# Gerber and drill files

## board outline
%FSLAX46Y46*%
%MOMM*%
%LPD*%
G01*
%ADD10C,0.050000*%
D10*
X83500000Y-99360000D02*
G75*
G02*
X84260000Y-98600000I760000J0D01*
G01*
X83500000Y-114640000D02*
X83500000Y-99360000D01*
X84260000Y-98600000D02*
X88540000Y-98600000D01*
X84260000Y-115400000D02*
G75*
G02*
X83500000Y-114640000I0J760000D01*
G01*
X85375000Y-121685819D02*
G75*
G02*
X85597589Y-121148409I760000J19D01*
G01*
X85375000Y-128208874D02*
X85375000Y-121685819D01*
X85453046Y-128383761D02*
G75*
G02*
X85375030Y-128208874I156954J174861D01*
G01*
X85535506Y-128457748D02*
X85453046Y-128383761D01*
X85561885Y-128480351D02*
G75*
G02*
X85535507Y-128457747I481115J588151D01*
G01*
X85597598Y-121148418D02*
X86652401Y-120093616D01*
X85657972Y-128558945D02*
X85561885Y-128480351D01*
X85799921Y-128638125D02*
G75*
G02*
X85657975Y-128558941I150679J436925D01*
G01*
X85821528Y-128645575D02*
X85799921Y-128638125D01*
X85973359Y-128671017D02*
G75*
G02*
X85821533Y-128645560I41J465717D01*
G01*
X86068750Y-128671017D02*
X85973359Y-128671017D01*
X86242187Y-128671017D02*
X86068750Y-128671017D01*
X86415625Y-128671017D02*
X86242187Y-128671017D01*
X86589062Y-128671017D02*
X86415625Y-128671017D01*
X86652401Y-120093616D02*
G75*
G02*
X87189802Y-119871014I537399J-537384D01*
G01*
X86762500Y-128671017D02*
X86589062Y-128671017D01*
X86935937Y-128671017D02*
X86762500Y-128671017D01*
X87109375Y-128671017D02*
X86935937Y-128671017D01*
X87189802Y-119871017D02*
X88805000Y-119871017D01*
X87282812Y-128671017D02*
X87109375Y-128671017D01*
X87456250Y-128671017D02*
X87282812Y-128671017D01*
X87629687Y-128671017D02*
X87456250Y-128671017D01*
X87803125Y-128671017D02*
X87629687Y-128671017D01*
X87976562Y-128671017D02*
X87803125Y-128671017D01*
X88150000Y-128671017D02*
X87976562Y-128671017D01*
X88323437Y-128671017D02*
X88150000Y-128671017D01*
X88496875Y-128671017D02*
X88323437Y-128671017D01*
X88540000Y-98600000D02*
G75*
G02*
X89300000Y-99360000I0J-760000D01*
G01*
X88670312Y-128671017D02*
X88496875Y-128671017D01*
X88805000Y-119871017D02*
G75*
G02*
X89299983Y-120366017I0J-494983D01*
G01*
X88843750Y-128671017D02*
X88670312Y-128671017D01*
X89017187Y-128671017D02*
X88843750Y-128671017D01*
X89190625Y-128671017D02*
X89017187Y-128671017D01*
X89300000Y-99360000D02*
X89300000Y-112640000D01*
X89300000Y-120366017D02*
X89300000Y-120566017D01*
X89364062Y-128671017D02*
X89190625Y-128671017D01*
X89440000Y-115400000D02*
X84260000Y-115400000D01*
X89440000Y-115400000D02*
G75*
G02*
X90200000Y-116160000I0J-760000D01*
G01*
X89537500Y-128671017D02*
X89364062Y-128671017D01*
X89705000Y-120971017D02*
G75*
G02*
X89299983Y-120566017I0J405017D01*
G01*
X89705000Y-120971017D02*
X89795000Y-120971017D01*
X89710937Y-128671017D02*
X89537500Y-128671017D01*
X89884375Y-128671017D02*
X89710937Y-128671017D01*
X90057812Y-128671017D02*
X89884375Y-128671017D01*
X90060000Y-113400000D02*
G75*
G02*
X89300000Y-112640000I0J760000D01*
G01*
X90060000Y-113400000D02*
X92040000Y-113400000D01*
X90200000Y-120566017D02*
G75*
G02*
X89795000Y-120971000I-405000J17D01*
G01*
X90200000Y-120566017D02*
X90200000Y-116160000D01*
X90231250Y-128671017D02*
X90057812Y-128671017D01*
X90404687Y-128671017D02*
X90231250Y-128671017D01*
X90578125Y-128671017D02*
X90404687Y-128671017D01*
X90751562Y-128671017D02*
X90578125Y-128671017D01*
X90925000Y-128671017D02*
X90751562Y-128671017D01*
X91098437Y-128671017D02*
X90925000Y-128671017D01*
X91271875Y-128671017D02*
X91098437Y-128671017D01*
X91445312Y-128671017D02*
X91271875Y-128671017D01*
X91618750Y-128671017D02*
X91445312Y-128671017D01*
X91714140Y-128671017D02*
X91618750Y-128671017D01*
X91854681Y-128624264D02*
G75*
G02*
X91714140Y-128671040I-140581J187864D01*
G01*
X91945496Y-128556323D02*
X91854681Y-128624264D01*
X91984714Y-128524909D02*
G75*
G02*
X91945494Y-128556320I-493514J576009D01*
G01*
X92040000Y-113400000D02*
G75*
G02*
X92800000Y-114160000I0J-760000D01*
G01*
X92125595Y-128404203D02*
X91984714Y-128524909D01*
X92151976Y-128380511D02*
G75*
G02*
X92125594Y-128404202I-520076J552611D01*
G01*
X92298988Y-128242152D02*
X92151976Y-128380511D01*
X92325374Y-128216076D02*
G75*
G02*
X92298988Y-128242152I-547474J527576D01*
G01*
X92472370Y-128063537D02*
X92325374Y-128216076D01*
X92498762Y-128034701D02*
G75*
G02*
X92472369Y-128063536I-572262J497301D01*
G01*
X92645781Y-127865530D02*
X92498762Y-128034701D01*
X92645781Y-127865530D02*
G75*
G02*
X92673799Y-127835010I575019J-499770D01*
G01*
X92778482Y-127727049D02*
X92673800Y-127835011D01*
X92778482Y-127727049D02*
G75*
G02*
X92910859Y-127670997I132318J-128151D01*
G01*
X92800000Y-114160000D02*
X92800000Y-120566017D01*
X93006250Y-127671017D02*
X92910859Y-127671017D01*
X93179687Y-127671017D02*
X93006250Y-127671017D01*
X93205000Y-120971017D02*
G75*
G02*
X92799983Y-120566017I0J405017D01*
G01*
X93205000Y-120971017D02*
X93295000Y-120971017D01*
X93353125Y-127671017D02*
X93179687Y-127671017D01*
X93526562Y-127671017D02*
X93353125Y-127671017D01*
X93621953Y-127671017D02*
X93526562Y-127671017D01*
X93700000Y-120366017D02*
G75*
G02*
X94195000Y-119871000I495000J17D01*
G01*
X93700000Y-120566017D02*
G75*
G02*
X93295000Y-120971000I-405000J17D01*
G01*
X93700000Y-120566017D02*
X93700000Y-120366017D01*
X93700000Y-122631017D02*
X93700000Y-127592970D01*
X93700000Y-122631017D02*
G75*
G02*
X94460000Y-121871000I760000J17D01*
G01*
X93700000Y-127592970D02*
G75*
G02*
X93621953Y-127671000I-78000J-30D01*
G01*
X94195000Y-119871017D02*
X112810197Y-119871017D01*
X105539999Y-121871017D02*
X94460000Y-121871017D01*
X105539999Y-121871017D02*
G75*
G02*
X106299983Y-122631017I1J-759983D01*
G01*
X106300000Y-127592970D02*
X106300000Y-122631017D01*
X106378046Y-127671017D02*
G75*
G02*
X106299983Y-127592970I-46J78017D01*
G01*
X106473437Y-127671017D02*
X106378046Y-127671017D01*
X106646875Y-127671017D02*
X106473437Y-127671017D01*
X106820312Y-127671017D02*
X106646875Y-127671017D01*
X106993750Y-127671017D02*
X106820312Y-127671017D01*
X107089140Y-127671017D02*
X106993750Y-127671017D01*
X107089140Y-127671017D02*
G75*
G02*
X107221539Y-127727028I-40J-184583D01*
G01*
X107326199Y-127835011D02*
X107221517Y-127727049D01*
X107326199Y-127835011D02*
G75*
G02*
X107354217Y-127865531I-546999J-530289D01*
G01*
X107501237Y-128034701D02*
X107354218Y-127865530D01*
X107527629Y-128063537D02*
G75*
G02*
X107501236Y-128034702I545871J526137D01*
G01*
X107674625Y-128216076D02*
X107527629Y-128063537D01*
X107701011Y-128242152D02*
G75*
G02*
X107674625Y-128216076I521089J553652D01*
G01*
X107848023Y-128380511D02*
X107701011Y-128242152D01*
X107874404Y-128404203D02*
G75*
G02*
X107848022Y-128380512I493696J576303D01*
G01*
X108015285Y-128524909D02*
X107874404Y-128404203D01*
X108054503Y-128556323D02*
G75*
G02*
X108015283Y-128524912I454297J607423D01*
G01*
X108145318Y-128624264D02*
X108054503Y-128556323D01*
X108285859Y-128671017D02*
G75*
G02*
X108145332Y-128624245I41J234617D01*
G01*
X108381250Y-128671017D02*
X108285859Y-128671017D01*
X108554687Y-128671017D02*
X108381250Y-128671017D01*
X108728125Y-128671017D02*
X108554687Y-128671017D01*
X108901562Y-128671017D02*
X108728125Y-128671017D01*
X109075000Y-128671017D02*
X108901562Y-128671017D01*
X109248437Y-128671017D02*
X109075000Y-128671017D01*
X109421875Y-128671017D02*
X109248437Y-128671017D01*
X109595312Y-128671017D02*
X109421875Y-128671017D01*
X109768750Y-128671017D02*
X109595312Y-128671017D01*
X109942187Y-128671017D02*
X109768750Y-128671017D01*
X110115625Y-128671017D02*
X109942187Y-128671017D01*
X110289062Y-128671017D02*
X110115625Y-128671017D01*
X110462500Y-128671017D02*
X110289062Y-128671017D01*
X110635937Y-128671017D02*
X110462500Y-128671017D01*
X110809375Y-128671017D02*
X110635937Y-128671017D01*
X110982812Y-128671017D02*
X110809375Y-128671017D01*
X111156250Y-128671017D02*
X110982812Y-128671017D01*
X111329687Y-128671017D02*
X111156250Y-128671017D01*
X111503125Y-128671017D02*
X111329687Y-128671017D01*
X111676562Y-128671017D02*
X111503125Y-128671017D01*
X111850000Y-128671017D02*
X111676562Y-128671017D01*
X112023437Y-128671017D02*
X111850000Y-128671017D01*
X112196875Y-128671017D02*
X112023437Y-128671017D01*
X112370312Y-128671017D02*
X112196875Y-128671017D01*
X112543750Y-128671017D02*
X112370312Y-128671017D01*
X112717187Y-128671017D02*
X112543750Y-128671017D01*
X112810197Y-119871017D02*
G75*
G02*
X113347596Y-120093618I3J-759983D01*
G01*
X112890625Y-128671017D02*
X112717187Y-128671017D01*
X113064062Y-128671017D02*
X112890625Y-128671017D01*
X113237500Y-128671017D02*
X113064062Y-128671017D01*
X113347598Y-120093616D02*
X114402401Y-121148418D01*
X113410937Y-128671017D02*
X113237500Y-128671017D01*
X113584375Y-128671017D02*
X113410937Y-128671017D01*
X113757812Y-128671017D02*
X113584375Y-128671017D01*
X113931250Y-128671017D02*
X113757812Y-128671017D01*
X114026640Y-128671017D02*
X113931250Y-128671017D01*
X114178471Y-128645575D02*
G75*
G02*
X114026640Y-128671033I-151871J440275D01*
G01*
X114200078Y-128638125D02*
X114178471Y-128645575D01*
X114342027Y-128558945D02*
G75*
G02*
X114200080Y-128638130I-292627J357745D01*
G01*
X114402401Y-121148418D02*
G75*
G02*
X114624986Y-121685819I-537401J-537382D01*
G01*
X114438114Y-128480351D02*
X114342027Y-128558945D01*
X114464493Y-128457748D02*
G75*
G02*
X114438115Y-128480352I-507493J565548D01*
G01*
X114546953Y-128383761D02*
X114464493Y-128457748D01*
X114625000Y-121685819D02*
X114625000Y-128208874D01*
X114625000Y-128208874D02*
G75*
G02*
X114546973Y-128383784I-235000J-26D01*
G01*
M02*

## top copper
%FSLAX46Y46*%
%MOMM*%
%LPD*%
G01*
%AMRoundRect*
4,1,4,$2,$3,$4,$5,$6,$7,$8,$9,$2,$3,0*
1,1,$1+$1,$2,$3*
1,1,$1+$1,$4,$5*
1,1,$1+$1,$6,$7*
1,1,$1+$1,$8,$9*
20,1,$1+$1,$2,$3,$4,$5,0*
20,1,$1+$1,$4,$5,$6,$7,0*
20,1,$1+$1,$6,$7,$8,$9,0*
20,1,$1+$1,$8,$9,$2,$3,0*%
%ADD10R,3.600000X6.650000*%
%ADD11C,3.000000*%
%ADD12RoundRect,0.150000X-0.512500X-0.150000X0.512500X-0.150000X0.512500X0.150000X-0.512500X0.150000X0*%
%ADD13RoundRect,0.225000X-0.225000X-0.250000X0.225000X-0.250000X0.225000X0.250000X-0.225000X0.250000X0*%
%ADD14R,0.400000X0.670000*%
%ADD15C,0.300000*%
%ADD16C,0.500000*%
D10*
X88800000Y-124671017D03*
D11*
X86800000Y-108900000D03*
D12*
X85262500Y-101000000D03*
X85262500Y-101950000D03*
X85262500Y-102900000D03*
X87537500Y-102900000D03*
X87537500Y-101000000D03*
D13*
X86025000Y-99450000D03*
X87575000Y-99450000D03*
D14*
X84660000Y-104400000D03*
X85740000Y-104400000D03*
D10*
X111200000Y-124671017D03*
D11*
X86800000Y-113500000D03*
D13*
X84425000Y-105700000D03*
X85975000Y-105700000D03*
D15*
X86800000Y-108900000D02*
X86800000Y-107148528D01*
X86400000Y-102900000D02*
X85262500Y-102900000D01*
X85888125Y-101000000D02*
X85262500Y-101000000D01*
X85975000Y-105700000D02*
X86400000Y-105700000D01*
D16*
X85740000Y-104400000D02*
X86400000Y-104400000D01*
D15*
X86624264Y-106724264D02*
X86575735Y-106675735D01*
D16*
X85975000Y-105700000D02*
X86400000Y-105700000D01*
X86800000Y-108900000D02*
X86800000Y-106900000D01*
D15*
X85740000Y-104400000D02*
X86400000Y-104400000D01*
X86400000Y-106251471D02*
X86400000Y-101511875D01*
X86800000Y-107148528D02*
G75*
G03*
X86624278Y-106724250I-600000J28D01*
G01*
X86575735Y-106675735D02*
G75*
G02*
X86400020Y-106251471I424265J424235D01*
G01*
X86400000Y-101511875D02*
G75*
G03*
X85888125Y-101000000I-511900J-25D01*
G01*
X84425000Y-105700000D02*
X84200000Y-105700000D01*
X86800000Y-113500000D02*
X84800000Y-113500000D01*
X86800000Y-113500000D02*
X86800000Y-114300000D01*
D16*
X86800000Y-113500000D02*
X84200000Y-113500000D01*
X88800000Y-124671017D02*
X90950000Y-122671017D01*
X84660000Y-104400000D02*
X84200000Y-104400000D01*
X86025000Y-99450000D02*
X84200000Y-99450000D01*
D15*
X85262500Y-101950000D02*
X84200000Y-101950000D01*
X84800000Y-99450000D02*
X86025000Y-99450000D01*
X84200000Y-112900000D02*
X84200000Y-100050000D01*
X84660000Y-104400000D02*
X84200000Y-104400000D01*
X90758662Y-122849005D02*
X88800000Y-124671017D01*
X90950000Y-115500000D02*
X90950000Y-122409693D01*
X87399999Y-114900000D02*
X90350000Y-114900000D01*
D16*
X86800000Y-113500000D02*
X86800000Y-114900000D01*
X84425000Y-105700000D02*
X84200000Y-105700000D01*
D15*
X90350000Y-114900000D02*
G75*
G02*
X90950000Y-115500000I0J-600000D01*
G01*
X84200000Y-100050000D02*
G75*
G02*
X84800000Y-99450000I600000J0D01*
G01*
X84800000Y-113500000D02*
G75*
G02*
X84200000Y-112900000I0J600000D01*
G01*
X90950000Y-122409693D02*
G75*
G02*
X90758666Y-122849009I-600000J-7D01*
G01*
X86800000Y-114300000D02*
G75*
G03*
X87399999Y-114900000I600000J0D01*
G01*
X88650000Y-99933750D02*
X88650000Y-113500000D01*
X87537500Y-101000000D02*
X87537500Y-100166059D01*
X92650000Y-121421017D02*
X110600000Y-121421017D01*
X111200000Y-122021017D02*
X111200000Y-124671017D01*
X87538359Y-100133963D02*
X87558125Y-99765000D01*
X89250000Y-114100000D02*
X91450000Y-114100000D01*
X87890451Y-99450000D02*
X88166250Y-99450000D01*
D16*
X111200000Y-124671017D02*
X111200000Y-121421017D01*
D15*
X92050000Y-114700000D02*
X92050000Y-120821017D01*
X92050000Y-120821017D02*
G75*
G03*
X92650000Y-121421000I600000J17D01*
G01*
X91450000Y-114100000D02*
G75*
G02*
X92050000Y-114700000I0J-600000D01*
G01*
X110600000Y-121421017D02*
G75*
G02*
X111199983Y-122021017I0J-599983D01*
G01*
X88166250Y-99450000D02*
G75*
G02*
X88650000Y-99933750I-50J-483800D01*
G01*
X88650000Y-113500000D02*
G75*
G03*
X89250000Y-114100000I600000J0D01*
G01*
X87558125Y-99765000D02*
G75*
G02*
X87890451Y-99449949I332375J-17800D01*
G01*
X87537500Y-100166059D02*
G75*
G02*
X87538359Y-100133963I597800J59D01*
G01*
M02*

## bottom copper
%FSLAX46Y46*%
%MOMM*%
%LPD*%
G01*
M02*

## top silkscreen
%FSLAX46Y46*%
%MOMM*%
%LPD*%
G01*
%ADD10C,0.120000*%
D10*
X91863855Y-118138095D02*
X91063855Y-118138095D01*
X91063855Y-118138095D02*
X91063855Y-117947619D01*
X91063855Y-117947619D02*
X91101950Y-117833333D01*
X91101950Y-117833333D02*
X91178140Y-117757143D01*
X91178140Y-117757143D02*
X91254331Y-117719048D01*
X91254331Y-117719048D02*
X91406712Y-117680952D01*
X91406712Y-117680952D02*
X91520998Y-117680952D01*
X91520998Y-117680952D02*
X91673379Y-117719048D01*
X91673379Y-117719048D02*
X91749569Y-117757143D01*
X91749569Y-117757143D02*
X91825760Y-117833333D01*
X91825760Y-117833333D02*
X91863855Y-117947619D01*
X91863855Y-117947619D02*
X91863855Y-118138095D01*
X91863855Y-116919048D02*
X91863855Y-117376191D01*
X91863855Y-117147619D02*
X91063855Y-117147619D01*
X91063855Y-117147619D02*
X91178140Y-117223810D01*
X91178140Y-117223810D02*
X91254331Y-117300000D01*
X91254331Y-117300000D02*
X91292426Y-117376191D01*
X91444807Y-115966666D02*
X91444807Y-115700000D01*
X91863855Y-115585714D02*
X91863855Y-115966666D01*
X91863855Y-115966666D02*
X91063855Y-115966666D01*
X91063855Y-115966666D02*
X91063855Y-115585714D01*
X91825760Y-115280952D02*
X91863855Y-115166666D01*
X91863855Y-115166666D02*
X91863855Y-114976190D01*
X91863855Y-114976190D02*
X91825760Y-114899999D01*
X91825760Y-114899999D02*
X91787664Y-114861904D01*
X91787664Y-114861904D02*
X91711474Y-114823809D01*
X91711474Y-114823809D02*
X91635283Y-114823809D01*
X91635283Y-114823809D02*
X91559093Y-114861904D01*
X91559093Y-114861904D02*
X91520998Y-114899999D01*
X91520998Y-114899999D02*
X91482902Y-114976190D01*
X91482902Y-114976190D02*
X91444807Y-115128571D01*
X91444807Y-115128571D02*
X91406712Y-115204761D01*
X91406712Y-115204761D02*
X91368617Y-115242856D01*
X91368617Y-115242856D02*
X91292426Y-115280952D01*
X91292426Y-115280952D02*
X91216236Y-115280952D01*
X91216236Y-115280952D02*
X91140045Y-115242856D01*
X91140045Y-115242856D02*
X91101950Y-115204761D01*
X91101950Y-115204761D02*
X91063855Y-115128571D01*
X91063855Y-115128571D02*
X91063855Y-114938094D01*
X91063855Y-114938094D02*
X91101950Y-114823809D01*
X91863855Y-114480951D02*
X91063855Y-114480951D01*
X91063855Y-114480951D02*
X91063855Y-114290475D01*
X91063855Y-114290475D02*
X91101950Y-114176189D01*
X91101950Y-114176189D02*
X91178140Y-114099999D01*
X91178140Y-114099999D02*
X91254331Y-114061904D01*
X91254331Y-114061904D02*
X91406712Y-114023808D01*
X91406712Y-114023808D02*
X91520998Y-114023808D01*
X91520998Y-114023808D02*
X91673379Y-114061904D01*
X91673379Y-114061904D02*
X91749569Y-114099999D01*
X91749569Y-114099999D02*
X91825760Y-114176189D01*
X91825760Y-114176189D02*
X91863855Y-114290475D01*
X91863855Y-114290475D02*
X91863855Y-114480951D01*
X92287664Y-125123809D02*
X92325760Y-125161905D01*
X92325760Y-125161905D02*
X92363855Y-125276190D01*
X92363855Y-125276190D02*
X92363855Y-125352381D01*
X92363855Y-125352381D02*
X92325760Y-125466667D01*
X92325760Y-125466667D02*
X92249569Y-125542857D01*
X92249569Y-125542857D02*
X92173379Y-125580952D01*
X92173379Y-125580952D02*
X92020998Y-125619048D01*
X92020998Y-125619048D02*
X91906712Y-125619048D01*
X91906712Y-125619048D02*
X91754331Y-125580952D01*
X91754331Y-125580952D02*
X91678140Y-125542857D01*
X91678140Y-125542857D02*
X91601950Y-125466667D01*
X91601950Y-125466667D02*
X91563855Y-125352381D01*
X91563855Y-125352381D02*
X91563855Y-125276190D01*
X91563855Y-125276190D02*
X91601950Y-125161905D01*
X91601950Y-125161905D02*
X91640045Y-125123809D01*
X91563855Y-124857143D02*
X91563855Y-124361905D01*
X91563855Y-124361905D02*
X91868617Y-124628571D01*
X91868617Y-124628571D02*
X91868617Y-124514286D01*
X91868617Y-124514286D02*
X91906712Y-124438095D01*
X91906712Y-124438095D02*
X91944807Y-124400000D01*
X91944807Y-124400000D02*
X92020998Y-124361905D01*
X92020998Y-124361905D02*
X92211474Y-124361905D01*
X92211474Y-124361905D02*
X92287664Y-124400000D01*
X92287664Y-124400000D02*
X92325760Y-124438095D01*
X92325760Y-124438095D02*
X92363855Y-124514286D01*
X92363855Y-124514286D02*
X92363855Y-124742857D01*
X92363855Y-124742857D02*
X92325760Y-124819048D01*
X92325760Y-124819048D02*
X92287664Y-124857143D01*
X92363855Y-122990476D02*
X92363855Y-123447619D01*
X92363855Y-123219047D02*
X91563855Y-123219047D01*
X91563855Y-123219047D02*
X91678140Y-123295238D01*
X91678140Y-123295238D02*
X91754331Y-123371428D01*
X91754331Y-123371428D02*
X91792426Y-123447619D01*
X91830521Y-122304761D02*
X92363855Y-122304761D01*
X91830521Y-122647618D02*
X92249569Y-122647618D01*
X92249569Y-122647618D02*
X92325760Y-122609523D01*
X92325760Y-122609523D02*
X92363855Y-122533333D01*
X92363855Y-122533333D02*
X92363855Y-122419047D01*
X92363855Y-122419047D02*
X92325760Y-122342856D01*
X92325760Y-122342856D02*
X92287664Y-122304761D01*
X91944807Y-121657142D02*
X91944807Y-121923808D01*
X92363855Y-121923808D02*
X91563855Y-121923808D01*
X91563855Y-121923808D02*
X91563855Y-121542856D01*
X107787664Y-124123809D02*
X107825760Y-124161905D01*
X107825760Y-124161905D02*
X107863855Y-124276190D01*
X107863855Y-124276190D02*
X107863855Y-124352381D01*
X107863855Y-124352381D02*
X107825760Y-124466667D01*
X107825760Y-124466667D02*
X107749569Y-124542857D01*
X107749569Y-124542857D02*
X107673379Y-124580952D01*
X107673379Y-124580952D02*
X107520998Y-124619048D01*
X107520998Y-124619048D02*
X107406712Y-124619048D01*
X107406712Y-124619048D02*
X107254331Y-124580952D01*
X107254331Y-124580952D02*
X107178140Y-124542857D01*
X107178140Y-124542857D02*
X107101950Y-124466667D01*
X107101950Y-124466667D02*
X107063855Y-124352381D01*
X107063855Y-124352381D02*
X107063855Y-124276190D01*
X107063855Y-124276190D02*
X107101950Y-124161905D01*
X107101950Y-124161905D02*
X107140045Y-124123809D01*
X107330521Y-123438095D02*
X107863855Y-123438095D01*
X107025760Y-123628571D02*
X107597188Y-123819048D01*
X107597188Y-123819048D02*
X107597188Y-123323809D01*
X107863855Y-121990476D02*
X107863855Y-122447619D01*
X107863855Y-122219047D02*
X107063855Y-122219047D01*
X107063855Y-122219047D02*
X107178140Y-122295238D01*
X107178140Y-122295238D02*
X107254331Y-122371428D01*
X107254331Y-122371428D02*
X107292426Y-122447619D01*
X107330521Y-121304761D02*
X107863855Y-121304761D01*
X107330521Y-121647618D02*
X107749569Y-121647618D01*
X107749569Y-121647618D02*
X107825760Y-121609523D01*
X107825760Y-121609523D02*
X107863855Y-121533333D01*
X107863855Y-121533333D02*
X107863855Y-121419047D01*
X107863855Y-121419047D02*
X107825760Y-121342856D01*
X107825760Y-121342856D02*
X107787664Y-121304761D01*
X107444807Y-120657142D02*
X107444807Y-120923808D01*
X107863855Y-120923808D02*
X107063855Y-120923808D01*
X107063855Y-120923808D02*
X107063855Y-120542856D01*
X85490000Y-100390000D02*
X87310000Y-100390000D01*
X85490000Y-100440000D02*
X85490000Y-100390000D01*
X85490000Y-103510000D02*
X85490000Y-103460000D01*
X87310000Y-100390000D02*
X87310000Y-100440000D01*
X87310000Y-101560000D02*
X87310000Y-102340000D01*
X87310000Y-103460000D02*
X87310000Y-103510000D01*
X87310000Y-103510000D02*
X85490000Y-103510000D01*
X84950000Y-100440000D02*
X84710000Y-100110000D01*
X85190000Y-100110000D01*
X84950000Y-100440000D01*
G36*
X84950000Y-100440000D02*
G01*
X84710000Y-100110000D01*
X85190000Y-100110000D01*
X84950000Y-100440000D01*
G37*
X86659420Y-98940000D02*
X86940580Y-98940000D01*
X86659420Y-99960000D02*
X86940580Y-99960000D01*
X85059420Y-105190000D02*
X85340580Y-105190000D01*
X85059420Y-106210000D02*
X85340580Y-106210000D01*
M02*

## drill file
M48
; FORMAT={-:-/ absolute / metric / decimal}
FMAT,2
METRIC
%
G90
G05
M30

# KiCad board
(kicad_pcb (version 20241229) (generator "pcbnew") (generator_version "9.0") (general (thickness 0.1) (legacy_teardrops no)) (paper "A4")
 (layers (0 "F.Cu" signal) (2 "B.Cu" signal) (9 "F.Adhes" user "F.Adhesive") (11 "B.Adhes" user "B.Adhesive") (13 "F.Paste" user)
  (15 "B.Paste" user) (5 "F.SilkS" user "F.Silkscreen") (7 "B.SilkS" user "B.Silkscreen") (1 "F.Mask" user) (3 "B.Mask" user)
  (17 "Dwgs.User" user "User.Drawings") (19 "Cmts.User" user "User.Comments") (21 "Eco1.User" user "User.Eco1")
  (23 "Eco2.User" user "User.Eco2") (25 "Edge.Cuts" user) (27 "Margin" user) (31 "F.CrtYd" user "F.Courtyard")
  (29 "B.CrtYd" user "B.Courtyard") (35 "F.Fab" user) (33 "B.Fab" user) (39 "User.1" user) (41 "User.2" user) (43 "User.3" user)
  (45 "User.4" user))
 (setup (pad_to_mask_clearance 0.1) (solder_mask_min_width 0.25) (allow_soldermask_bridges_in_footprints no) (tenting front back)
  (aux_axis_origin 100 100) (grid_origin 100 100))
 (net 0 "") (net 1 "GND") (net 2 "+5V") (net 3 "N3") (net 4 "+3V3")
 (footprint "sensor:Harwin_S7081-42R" (layer "F.Cu") (at 88.8 124.671017 90)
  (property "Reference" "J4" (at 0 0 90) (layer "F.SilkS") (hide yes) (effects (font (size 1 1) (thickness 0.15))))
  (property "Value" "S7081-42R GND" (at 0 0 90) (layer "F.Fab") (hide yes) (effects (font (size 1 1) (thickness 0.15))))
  (pad "1" smd rect (at 0 0 90) (size 6.65 3.6) (layers "F.Cu" "F.Mask" "F.Paste") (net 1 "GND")))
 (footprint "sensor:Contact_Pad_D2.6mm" (layer "F.Cu") (at 86.8 108.9)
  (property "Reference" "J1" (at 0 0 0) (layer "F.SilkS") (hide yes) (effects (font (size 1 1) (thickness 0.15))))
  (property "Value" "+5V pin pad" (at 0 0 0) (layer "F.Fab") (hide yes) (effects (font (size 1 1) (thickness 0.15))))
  (pad "1" smd circle (at 0 0) (size 3 3) (layers "F.Cu" "F.Mask") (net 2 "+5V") (solder_mask_margin -0.2)))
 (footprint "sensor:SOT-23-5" (layer "F.Cu") (at 86.4 101.95)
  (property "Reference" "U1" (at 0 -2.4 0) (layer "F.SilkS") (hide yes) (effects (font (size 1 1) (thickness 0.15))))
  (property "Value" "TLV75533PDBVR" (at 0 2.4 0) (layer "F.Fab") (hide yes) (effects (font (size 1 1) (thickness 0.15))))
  (fp_line (start -0.91 -1.56) (end 0.91 -1.56) (stroke (width 0.12) (type solid)) (layer "F.SilkS"))
  (fp_line (start -0.91 -1.51) (end -0.91 -1.56) (stroke (width 0.12) (type solid)) (layer "F.SilkS"))
  (fp_line (start -0.91 1.56) (end -0.91 1.51) (stroke (width 0.12) (type solid)) (layer "F.SilkS"))
  (fp_line (start 0.91 -1.56) (end 0.91 -1.51) (stroke (width 0.12) (type solid)) (layer "F.SilkS"))
  (fp_line (start 0.91 -0.39) (end 0.91 0.39) (stroke (width 0.12) (type solid)) (layer "F.SilkS"))
  (fp_line (start 0.91 1.51) (end 0.91 1.56) (stroke (width 0.12) (type solid)) (layer "F.SilkS"))
  (fp_line (start 0.91 1.56) (end -0.91 1.56) (stroke (width 0.12) (type solid)) (layer "F.SilkS"))
  (fp_poly (pts (xy -1.45 -1.51) (xy -1.69 -1.84) (xy -1.21 -1.84)) (stroke (width 0.12) (type solid)) (fill yes) (layer "F.SilkS"))
  (pad "1" smd roundrect (at -1.1375 -0.95) (size 1.325 0.6) (layers "F.Cu" "F.Mask" "F.Paste") (roundrect_rratio 0.25) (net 2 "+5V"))
  (pad "2" smd roundrect (at -1.1375 0) (size 1.325 0.6) (layers "F.Cu" "F.Mask" "F.Paste") (roundrect_rratio 0.25) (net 1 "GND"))
  (pad "3" smd roundrect (at -1.1375 0.95) (size 1.325 0.6) (layers "F.Cu" "F.Mask" "F.Paste") (roundrect_rratio 0.25) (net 2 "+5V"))
  (pad "4" smd roundrect (at 1.1375 0.95) (size 1.325 0.6) (layers "F.Cu" "F.Mask" "F.Paste") (roundrect_rratio 0.25) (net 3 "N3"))
  (pad "5" smd roundrect (at 1.1375 -0.95) (size 1.325 0.6) (layers "F.Cu" "F.Mask" "F.Paste") (roundrect_rratio 0.25) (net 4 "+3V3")))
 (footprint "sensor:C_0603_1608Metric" (layer "F.Cu") (at 86.8 99.45)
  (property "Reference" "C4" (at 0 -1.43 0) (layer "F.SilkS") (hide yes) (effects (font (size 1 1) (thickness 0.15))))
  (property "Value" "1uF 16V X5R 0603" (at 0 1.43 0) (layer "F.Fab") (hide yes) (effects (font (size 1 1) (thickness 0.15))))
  (fp_line (start -0.14058 -0.51) (end 0.14058 -0.51) (stroke (width 0.12) (type solid)) (layer "F.SilkS"))
  (fp_line (start -0.14058 0.51) (end 0.14058 0.51) (stroke (width 0.12) (type solid)) (layer "F.SilkS"))
  (pad "1" smd roundrect (at -0.775 0) (size 0.9 0.95) (layers "F.Cu" "F.Mask" "F.Paste") (roundrect_rratio 0.25) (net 1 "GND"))
  (pad "2" smd roundrect (at 0.775 0) (size 0.9 0.95) (layers "F.Cu" "F.Mask" "F.Paste") (roundrect_rratio 0.25) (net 4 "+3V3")))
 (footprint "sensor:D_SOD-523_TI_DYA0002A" (layer "F.Cu") (at 85.2 104.4)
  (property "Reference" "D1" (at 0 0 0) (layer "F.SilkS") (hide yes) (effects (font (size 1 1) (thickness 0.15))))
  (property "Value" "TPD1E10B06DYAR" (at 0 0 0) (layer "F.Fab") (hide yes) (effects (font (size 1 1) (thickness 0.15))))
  (pad "1" smd rect (at -0.54 0) (size 0.4 0.67) (layers "F.Cu" "F.Mask" "F.Paste") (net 1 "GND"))
  (pad "2" smd rect (at 0.54 0) (size 0.4 0.67) (layers "F.Cu" "F.Mask" "F.Paste") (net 2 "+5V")))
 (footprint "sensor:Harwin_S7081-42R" (layer "F.Cu") (at 111.2 124.671017 90)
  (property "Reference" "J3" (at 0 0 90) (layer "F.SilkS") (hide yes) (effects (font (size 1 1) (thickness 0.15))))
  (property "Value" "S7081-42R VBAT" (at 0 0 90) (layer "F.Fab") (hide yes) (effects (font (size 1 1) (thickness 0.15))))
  (pad "1" smd rect (at 0 0 90) (size 6.65 3.6) (layers "F.Cu" "F.Mask" "F.Paste") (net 4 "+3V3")))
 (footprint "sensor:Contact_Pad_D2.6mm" (layer "F.Cu") (at 86.8 113.5)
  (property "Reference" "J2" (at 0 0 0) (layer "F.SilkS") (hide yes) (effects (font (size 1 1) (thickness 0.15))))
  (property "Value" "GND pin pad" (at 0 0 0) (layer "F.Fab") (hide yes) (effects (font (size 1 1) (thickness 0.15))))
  (pad "1" smd circle (at 0 0) (size 3 3) (layers "F.Cu" "F.Mask") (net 1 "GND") (solder_mask_margin -0.2)))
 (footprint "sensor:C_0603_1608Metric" (layer "F.Cu") (at 85.2 105.7)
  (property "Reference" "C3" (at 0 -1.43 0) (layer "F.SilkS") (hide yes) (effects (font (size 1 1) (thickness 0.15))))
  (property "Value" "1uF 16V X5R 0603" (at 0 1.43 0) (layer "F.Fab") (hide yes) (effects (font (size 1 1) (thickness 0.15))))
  (fp_line (start -0.14058 -0.51) (end 0.14058 -0.51) (stroke (width 0.12) (type solid)) (layer "F.SilkS"))
  (fp_line (start -0.14058 0.51) (end 0.14058 0.51) (stroke (width 0.12) (type solid)) (layer "F.SilkS"))
  (pad "1" smd roundrect (at -0.775 0) (size 0.9 0.95) (layers "F.Cu" "F.Mask" "F.Paste") (roundrect_rratio 0.25) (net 1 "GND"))
  (pad "2" smd roundrect (at 0.775 0) (size 0.9 0.95) (layers "F.Cu" "F.Mask" "F.Paste") (roundrect_rratio 0.25) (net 2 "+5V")))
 (gr_arc (start 83.5 99.36) (mid 83.722598 98.822598) (end 84.26 98.6) (stroke (width 0.05) (type default)) (layer "Edge.Cuts"))
 (gr_line (start 83.5 114.64) (end 83.5 99.36) (stroke (width 0.05) (type default)) (layer "Edge.Cuts"))
 (gr_line (start 84.26 98.6) (end 88.54 98.6) (stroke (width 0.05) (type default)) (layer "Edge.Cuts"))
 (gr_arc (start 84.26 115.4) (mid 83.722598 115.177401) (end 83.5 114.64) (stroke (width 0.05) (type default)) (layer "Edge.Cuts"))
 (gr_arc (start 85.375 121.685819) (mid 85.432851 121.39498) (end 85.597598 121.148418) (stroke (width 0.05) (type default))
  (layer "Edge.Cuts"))
 (gr_line (start 85.375 128.208874) (end 85.375 121.685819) (stroke (width 0.05) (type default)) (layer "Edge.Cuts"))
 (gr_arc (start 85.453046 128.383761) (mid 85.395397 128.30463) (end 85.375 128.208874) (stroke (width 0.05) (type default))
  (layer "Edge.Cuts"))
 (gr_line (start 85.535506 128.457748) (end 85.453046 128.383761) (stroke (width 0.05) (type default)) (layer "Edge.Cuts"))
 (gr_arc (start 85.561885 128.480351) (mid 85.548566 128.4692) (end 85.535506 128.457748) (stroke (width 0.05) (type default))
  (layer "Edge.Cuts"))
 (gr_line (start 85.597598 121.148418) (end 86.652401 120.093616) (stroke (width 0.05) (type default)) (layer "Edge.Cuts"))
 (gr_line (start 85.657972 128.558945) (end 85.561885 128.480351) (stroke (width 0.05) (type default)) (layer "Edge.Cuts"))
 (gr_arc (start 85.799921 128.638125) (mid 85.725438 128.604824) (end 85.657972 128.558945) (stroke (width 0.05) (type default))
  (layer "Edge.Cuts"))
 (gr_line (start 85.821528 128.645575) (end 85.799921 128.638125) (stroke (width 0.05) (type default)) (layer "Edge.Cuts"))
 (gr_arc (start 85.973359 128.671017) (mid 85.896385 128.664613) (end 85.821528 128.645575) (stroke (width 0.05) (type default))
  (layer "Edge.Cuts"))
 (gr_line (start 86.06875 128.671017) (end 85.973359 128.671017) (stroke (width 0.05) (type default)) (layer "Edge.Cuts"))
 (gr_line (start 86.242187 128.671017) (end 86.06875 128.671017) (stroke (width 0.05) (type default)) (layer "Edge.Cuts"))
 (gr_line (start 86.415625 128.671017) (end 86.242187 128.671017) (stroke (width 0.05) (type default)) (layer "Edge.Cuts"))
 (gr_line (start 86.589062 128.671017) (end 86.415625 128.671017) (stroke (width 0.05) (type default)) (layer "Edge.Cuts"))
 (gr_arc (start 86.652401 120.093616) (mid 86.898962 119.928869) (end 87.189802 119.871017) (stroke (width 0.05) (type default))
  (layer "Edge.Cuts"))
 (gr_line (start 86.7625 128.671017) (end 86.589062 128.671017) (stroke (width 0.05) (type default)) (layer "Edge.Cuts"))
 (gr_line (start 86.935937 128.671017) (end 86.7625 128.671017) (stroke (width 0.05) (type default)) (layer "Edge.Cuts"))
 (gr_line (start 87.109375 128.671017) (end 86.935937 128.671017) (stroke (width 0.05) (type default)) (layer "Edge.Cuts"))
 (gr_line (start 87.189802 119.871017) (end 88.805 119.871017) (stroke (width 0.05) (type default)) (layer "Edge.Cuts"))
 (gr_line (start 87.282812 128.671017) (end 87.109375 128.671017) (stroke (width 0.05) (type default)) (layer "Edge.Cuts"))
 (gr_line (start 87.45625 128.671017) (end 87.282812 128.671017) (stroke (width 0.05) (type default)) (layer "Edge.Cuts"))
 (gr_line (start 87.629687 128.671017) (end 87.45625 128.671017) (stroke (width 0.05) (type default)) (layer "Edge.Cuts"))
 (gr_line (start 87.803125 128.671017) (end 87.629687 128.671017) (stroke (width 0.05) (type default)) (layer "Edge.Cuts"))
 (gr_line (start 87.976562 128.671017) (end 87.803125 128.671017) (stroke (width 0.05) (type default)) (layer "Edge.Cuts"))
 (gr_line (start 88.15 128.671017) (end 87.976562 128.671017) (stroke (width 0.05) (type default)) (layer "Edge.Cuts"))
 (gr_line (start 88.323437 128.671017) (end 88.15 128.671017) (stroke (width 0.05) (type default)) (layer "Edge.Cuts"))
 (gr_line (start 88.496875 128.671017) (end 88.323437 128.671017) (stroke (width 0.05) (type default)) (layer "Edge.Cuts"))
 (gr_arc (start 88.54 98.6) (mid 89.077401 98.822598) (end 89.3 99.36) (stroke (width 0.05) (type default)) (layer "Edge.Cuts"))
 (gr_line (start 88.670312 128.671017) (end 88.496875 128.671017) (stroke (width 0.05) (type default)) (layer "Edge.Cuts"))
 (gr_arc (start 88.805 119.871017) (mid 89.155017 120.015999) (end 89.3 120.366017) (stroke (width 0.05) (type default)) (layer "Edge.Cuts"))
 (gr_line (start 88.84375 128.671017) (end 88.670312 128.671017) (stroke (width 0.05) (type default)) (layer "Edge.Cuts"))
 (gr_line (start 89.017187 128.671017) (end 88.84375 128.671017) (stroke (width 0.05) (type default)) (layer "Edge.Cuts"))
 (gr_line (start 89.190625 128.671017) (end 89.017187 128.671017) (stroke (width 0.05) (type default)) (layer "Edge.Cuts"))
 (gr_line (start 89.3 99.36) (end 89.3 112.64) (stroke (width 0.05) (type default)) (layer "Edge.Cuts"))
 (gr_line (start 89.3 120.366017) (end 89.3 120.566017) (stroke (width 0.05) (type default)) (layer "Edge.Cuts"))
 (gr_line (start 89.364062 128.671017) (end 89.190625 128.671017) (stroke (width 0.05) (type default)) (layer "Edge.Cuts"))
 (gr_line (start 89.44 115.4) (end 84.26 115.4) (stroke (width 0.05) (type default)) (layer "Edge.Cuts"))
 (gr_arc (start 89.44 115.4) (mid 89.977401 115.622599) (end 90.2 116.16) (stroke (width 0.05) (type default)) (layer "Edge.Cuts"))
 (gr_line (start 89.5375 128.671017) (end 89.364062 128.671017) (stroke (width 0.05) (type default)) (layer "Edge.Cuts"))
 (gr_arc (start 89.705 120.971017) (mid 89.418616 120.852396) (end 89.3 120.566017) (stroke (width 0.05) (type default)) (layer "Edge.Cuts"))
 (gr_line (start 89.705 120.971017) (end 89.795 120.971017) (stroke (width 0.05) (type default)) (layer "Edge.Cuts"))
 (gr_line (start 89.710937 128.671017) (end 89.5375 128.671017) (stroke (width 0.05) (type default)) (layer "Edge.Cuts"))
 (gr_line (start 89.884375 128.671017) (end 89.710937 128.671017) (stroke (width 0.05) (type default)) (layer "Edge.Cuts"))
 (gr_line (start 90.057812 128.671017) (end 89.884375 128.671017) (stroke (width 0.05) (type default)) (layer "Edge.Cuts"))
 (gr_arc (start 90.06 113.4) (mid 89.522599 113.177401) (end 89.3 112.64) (stroke (width 0.05) (type default)) (layer "Edge.Cuts"))
 (gr_line (start 90.06 113.4) (end 92.04 113.4) (stroke (width 0.05) (type default)) (layer "Edge.Cuts"))
 (gr_arc (start 90.2 120.566017) (mid 90.081372 120.852384) (end 89.795 120.971017) (stroke (width 0.05) (type default)) (layer "Edge.Cuts"))
 (gr_line (start 90.2 120.566017) (end 90.2 116.16) (stroke (width 0.05) (type default)) (layer "Edge.Cuts"))
 (gr_line (start 90.23125 128.671017) (end 90.057812 128.671017) (stroke (width 0.05) (type default)) (layer "Edge.Cuts"))
 (gr_line (start 90.404687 128.671017) (end 90.23125 128.671017) (stroke (width 0.05) (type default)) (layer "Edge.Cuts"))
 (gr_line (start 90.578125 128.671017) (end 90.404687 128.671017) (stroke (width 0.05) (type default)) (layer "Edge.Cuts"))
 (gr_line (start 90.751562 128.671017) (end 90.578125 128.671017) (stroke (width 0.05) (type default)) (layer "Edge.Cuts"))
 (gr_line (start 90.925 128.671017) (end 90.751562 128.671017) (stroke (width 0.05) (type default)) (layer "Edge.Cuts"))
 (gr_line (start 91.098437 128.671017) (end 90.925 128.671017) (stroke (width 0.05) (type default)) (layer "Edge.Cuts"))
 (gr_line (start 91.271875 128.671017) (end 91.098437 128.671017) (stroke (width 0.05) (type default)) (layer "Edge.Cuts"))
 (gr_line (start 91.445312 128.671017) (end 91.271875 128.671017) (stroke (width 0.05) (type default)) (layer "Edge.Cuts"))
 (gr_line (start 91.61875 128.671017) (end 91.445312 128.671017) (stroke (width 0.05) (type default)) (layer "Edge.Cuts"))
 (gr_line (start 91.71414 128.671017) (end 91.61875 128.671017) (stroke (width 0.05) (type default)) (layer "Edge.Cuts"))
 (gr_arc (start 91.854681 128.624264) (mid 91.788197 128.659022) (end 91.71414 128.671017) (stroke (width 0.05) (type default))
  (layer "Edge.Cuts"))
 (gr_line (start 91.945496 128.556323) (end 91.854681 128.624264) (stroke (width 0.05) (type default)) (layer "Edge.Cuts"))
 (gr_arc (start 91.984714 128.524909) (mid 91.965365 128.540941) (end 91.945496 128.556323) (stroke (width 0.05) (type default))
  (layer "Edge.Cuts"))
 (gr_arc (start 92.04 113.4) (mid 92.577401 113.622598) (end 92.8 114.16) (stroke (width 0.05) (type default)) (layer "Edge.Cuts"))
 (gr_line (start 92.125595 128.404203) (end 91.984714 128.524909) (stroke (width 0.05) (type default)) (layer "Edge.Cuts"))
 (gr_arc (start 92.151976 128.380511) (mid 92.138924 128.392511) (end 92.125595 128.404203) (stroke (width 0.05) (type default))
  (layer "Edge.Cuts"))
 (gr_line (start 92.298988 128.242152) (end 92.151976 128.380511) (stroke (width 0.05) (type default)) (layer "Edge.Cuts"))
 (gr_arc (start 92.325374 128.216076) (mid 92.31234 128.229275) (end 92.298988 128.242152) (stroke (width 0.05) (type default))
  (layer "Edge.Cuts"))
 (gr_line (start 92.47237 128.063537) (end 92.325374 128.216076) (stroke (width 0.05) (type default)) (layer "Edge.Cuts"))
 (gr_arc (start 92.498762 128.034701) (mid 92.485752 128.049289) (end 92.47237 128.063537) (stroke (width 0.05) (type default))
  (layer "Edge.Cuts"))
 (gr_line (start 92.645781 127.86553) (end 92.498762 128.034701) (stroke (width 0.05) (type default)) (layer "Edge.Cuts"))
 (gr_arc (start 92.645781 127.86553) (mid 92.659583 127.85008) (end 92.6738 127.835011) (stroke (width 0.05) (type default))
  (layer "Edge.Cuts"))
 (gr_line (start 92.778482 127.727049) (end 92.6738 127.835011) (stroke (width 0.05) (type default)) (layer "Edge.Cuts"))
 (gr_arc (start 92.778482 127.727049) (mid 92.838983 127.685587) (end 92.910859 127.671017) (stroke (width 0.05) (type default))
  (layer "Edge.Cuts"))
 (gr_line (start 92.8 114.16) (end 92.8 120.566017) (stroke (width 0.05) (type default)) (layer "Edge.Cuts"))
 (gr_line (start 93.00625 127.671017) (end 92.910859 127.671017) (stroke (width 0.05) (type default)) (layer "Edge.Cuts"))
 (gr_line (start 93.179687 127.671017) (end 93.00625 127.671017) (stroke (width 0.05) (type default)) (layer "Edge.Cuts"))
 (gr_arc (start 93.205 120.971017) (mid 92.918616 120.852396) (end 92.8 120.566017) (stroke (width 0.05) (type default)) (layer "Edge.Cuts"))
 (gr_line (start 93.205 120.971017) (end 93.295 120.971017) (stroke (width 0.05) (type default)) (layer "Edge.Cuts"))
 (gr_line (start 93.353125 127.671017) (end 93.179687 127.671017) (stroke (width 0.05) (type default)) (layer "Edge.Cuts"))
 (gr_line (start 93.526562 127.671017) (end 93.353125 127.671017) (stroke (width 0.05) (type default)) (layer "Edge.Cuts"))
 (gr_line (start 93.621953 127.671017) (end 93.526562 127.671017) (stroke (width 0.05) (type default)) (layer "Edge.Cuts"))
 (gr_arc (start 93.7 120.366017) (mid 93.844982 120.015999) (end 94.195 119.871017) (stroke (width 0.05) (type default)) (layer "Edge.Cuts"))
 (gr_arc (start 93.7 120.566017) (mid 93.581372 120.852384) (end 93.295 120.971017) (stroke (width 0.05) (type default)) (layer "Edge.Cuts"))
 (gr_line (start 93.7 120.566017) (end 93.7 120.366017) (stroke (width 0.05) (type default)) (layer "Edge.Cuts"))
 (gr_line (start 93.7 122.631017) (end 93.7 127.59297) (stroke (width 0.05) (type default)) (layer "Edge.Cuts"))
 (gr_arc (start 93.7 122.631017) (mid 93.922593 122.093605) (end 94.46 121.871017) (stroke (width 0.05) (type default)) (layer "Edge.Cuts"))
 (gr_arc (start 93.7 127.59297) (mid 93.67714 127.648158) (end 93.621953 127.671017) (stroke (width 0.05) (type default))
  (layer "Edge.Cuts"))
 (gr_line (start 94.195 119.871017) (end 112.810197 119.871017) (stroke (width 0.05) (type default)) (layer "Edge.Cuts"))
 (gr_line (start 105.539999 121.871017) (end 94.46 121.871017) (stroke (width 0.05) (type default)) (layer "Edge.Cuts"))
 (gr_arc (start 105.539999 121.871017) (mid 106.077395 122.093617) (end 106.3 122.631017) (stroke (width 0.05) (type default))
  (layer "Edge.Cuts"))
 (gr_line (start 106.3 127.59297) (end 106.3 122.631017) (stroke (width 0.05) (type default)) (layer "Edge.Cuts"))
 (gr_arc (start 106.378046 127.671017) (mid 106.322859 127.648158) (end 106.3 127.59297) (stroke (width 0.05) (type default))
  (layer "Edge.Cuts"))
 (gr_line (start 106.473437 127.671017) (end 106.378046 127.671017) (stroke (width 0.05) (type default)) (layer "Edge.Cuts"))
 (gr_line (start 106.646875 127.671017) (end 106.473437 127.671017) (stroke (width 0.05) (type default)) (layer "Edge.Cuts"))
 (gr_line (start 106.820312 127.671017) (end 106.646875 127.671017) (stroke (width 0.05) (type default)) (layer "Edge.Cuts"))
 (gr_line (start 106.99375 127.671017) (end 106.820312 127.671017) (stroke (width 0.05) (type default)) (layer "Edge.Cuts"))
 (gr_line (start 107.08914 127.671017) (end 106.99375 127.671017) (stroke (width 0.05) (type default)) (layer "Edge.Cuts"))
 (gr_arc (start 107.08914 127.671017) (mid 107.161005 127.685615) (end 107.221517 127.727049) (stroke (width 0.05) (type default))
  (layer "Edge.Cuts"))
 (gr_line (start 107.326199 127.835011) (end 107.221517 127.727049) (stroke (width 0.05) (type default)) (layer "Edge.Cuts"))
 (gr_arc (start 107.326199 127.835011) (mid 107.340416 127.85008) (end 107.354218 127.86553) (stroke (width 0.05) (type default))
  (layer "Edge.Cuts"))
 (gr_line (start 107.501237 128.034701) (end 107.354218 127.86553) (stroke (width 0.05) (type default)) (layer "Edge.Cuts"))
 (gr_arc (start 107.527629 128.063537) (mid 107.514247 128.049289) (end 107.501237 128.034701) (stroke (width 0.05) (type default))
  (layer "Edge.Cuts"))
 (gr_line (start 107.674625 128.216076) (end 107.527629 128.063537) (stroke (width 0.05) (type default)) (layer "Edge.Cuts"))
 (gr_arc (start 107.701011 128.242152) (mid 107.687659 128.229275) (end 107.674625 128.216076) (stroke (width 0.05) (type default))
  (layer "Edge.Cuts"))
 (gr_line (start 107.848023 128.380511) (end 107.701011 128.242152) (stroke (width 0.05) (type default)) (layer "Edge.Cuts"))
 (gr_arc (start 107.874404 128.404203) (mid 107.861075 128.392511) (end 107.848023 128.380511) (stroke (width 0.05) (type default))
  (layer "Edge.Cuts"))
 (gr_line (start 108.015285 128.524909) (end 107.874404 128.404203) (stroke (width 0.05) (type default)) (layer "Edge.Cuts"))
 (gr_arc (start 108.054503 128.556323) (mid 108.034634 128.540941) (end 108.015285 128.524909) (stroke (width 0.05) (type default))
  (layer "Edge.Cuts"))
 (gr_line (start 108.145318 128.624264) (end 108.054503 128.556323) (stroke (width 0.05) (type default)) (layer "Edge.Cuts"))
 (gr_arc (start 108.285859 128.671017) (mid 108.211802 128.659022) (end 108.145318 128.624264) (stroke (width 0.05) (type default))
  (layer "Edge.Cuts"))
 (gr_line (start 108.38125 128.671017) (end 108.285859 128.671017) (stroke (width 0.05) (type default)) (layer "Edge.Cuts"))
 (gr_line (start 108.554687 128.671017) (end 108.38125 128.671017) (stroke (width 0.05) (type default)) (layer "Edge.Cuts"))
 (gr_line (start 108.728125 128.671017) (end 108.554687 128.671017) (stroke (width 0.05) (type default)) (layer "Edge.Cuts"))
 (gr_line (start 108.901562 128.671017) (end 108.728125 128.671017) (stroke (width 0.05) (type default)) (layer "Edge.Cuts"))
 (gr_line (start 109.075 128.671017) (end 108.901562 128.671017) (stroke (width 0.05) (type default)) (layer "Edge.Cuts"))
 (gr_line (start 109.248437 128.671017) (end 109.075 128.671017) (stroke (width 0.05) (type default)) (layer "Edge.Cuts"))
 (gr_line (start 109.421875 128.671017) (end 109.248437 128.671017) (stroke (width 0.05) (type default)) (layer "Edge.Cuts"))
 (gr_line (start 109.595312 128.671017) (end 109.421875 128.671017) (stroke (width 0.05) (type default)) (layer "Edge.Cuts"))
 (gr_line (start 109.76875 128.671017) (end 109.595312 128.671017) (stroke (width 0.05) (type default)) (layer "Edge.Cuts"))
 (gr_line (start 109.942187 128.671017) (end 109.76875 128.671017) (stroke (width 0.05) (type default)) (layer "Edge.Cuts"))
 (gr_line (start 110.115625 128.671017) (end 109.942187 128.671017) (stroke (width 0.05) (type default)) (layer "Edge.Cuts"))
 (gr_line (start 110.289062 128.671017) (end 110.115625 128.671017) (stroke (width 0.05) (type default)) (layer "Edge.Cuts"))
 (gr_line (start 110.4625 128.671017) (end 110.289062 128.671017) (stroke (width 0.05) (type default)) (layer "Edge.Cuts"))
 (gr_line (start 110.635937 128.671017) (end 110.4625 128.671017) (stroke (width 0.05) (type default)) (layer "Edge.Cuts"))
 (gr_line (start 110.809375 128.671017) (end 110.635937 128.671017) (stroke (width 0.05) (type default)) (layer "Edge.Cuts"))
 (gr_line (start 110.982812 128.671017) (end 110.809375 128.671017) (stroke (width 0.05) (type default)) (layer "Edge.Cuts"))
 (gr_line (start 111.15625 128.671017) (end 110.982812 128.671017) (stroke (width 0.05) (type default)) (layer "Edge.Cuts"))
 (gr_line (start 111.329687 128.671017) (end 111.15625 128.671017) (stroke (width 0.05) (type default)) (layer "Edge.Cuts"))
 (gr_line (start 111.503125 128.671017) (end 111.329687 128.671017) (stroke (width 0.05) (type default)) (layer "Edge.Cuts"))
 (gr_line (start 111.676562 128.671017) (end 111.503125 128.671017) (stroke (width 0.05) (type default)) (layer "Edge.Cuts"))
 (gr_line (start 111.85 128.671017) (end 111.676562 128.671017) (stroke (width 0.05) (type default)) (layer "Edge.Cuts"))
 (gr_line (start 112.023437 128.671017) (end 111.85 128.671017) (stroke (width 0.05) (type default)) (layer "Edge.Cuts"))
 (gr_line (start 112.196875 128.671017) (end 112.023437 128.671017) (stroke (width 0.05) (type default)) (layer "Edge.Cuts"))
 (gr_line (start 112.370312 128.671017) (end 112.196875 128.671017) (stroke (width 0.05) (type default)) (layer "Edge.Cuts"))
 (gr_line (start 112.54375 128.671017) (end 112.370312 128.671017) (stroke (width 0.05) (type default)) (layer "Edge.Cuts"))
 (gr_line (start 112.717187 128.671017) (end 112.54375 128.671017) (stroke (width 0.05) (type default)) (layer "Edge.Cuts"))
 (gr_arc (start 112.810197 119.871017) (mid 113.101037 119.928869) (end 113.347598 120.093616) (stroke (width 0.05) (type default))
  (layer "Edge.Cuts"))
 (gr_line (start 112.890625 128.671017) (end 112.717187 128.671017) (stroke (width 0.05) (type default)) (layer "Edge.Cuts"))
 (gr_line (start 113.064062 128.671017) (end 112.890625 128.671017) (stroke (width 0.05) (type default)) (layer "Edge.Cuts"))
 (gr_line (start 113.2375 128.671017) (end 113.064062 128.671017) (stroke (width 0.05) (type default)) (layer "Edge.Cuts"))
 (gr_line (start 113.347598 120.093616) (end 114.402401 121.148418) (stroke (width 0.05) (type default)) (layer "Edge.Cuts"))
 (gr_line (start 113.410937 128.671017) (end 113.2375 128.671017) (stroke (width 0.05) (type default)) (layer "Edge.Cuts"))
 (gr_line (start 113.584375 128.671017) (end 113.410937 128.671017) (stroke (width 0.05) (type default)) (layer "Edge.Cuts"))
 (gr_line (start 113.757812 128.671017) (end 113.584375 128.671017) (stroke (width 0.05) (type default)) (layer "Edge.Cuts"))
 (gr_line (start 113.93125 128.671017) (end 113.757812 128.671017) (stroke (width 0.05) (type default)) (layer "Edge.Cuts"))
 (gr_line (start 114.02664 128.671017) (end 113.93125 128.671017) (stroke (width 0.05) (type default)) (layer "Edge.Cuts"))
 (gr_arc (start 114.178471 128.645575) (mid 114.103614 128.664613) (end 114.02664 128.671017) (stroke (width 0.05) (type default))
  (layer "Edge.Cuts"))
 (gr_line (start 114.200078 128.638125) (end 114.178471 128.645575) (stroke (width 0.05) (type default)) (layer "Edge.Cuts"))
 (gr_arc (start 114.342027 128.558945) (mid 114.274561 128.604824) (end 114.200078 128.638125) (stroke (width 0.05) (type default))
  (layer "Edge.Cuts"))
 (gr_arc (start 114.402401 121.148418) (mid 114.567148 121.39498) (end 114.625 121.685819) (stroke (width 0.05) (type default))
  (layer "Edge.Cuts"))
 (gr_line (start 114.438114 128.480351) (end 114.342027 128.558945) (stroke (width 0.05) (type default)) (layer "Edge.Cuts"))
 (gr_arc (start 114.464493 128.457748) (mid 114.451433 128.4692) (end 114.438114 128.480351) (stroke (width 0.05) (type default))
  (layer "Edge.Cuts"))
 (gr_line (start 114.546953 128.383761) (end 114.464493 128.457748) (stroke (width 0.05) (type default)) (layer "Edge.Cuts"))
 (gr_line (start 114.625 121.685819) (end 114.625 128.208874) (stroke (width 0.05) (type default)) (layer "Edge.Cuts"))
 (gr_arc (start 114.625 128.208874) (mid 114.604602 128.30463) (end 114.546953 128.383761) (stroke (width 0.05) (type default))
  (layer "Edge.Cuts"))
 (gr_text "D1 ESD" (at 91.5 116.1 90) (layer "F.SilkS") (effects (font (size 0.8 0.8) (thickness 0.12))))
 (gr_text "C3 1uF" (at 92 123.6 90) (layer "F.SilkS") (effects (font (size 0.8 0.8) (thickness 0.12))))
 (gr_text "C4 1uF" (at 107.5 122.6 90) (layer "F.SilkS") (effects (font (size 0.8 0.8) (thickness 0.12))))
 (segment (start 86.8 108.9) (end 86.8 107.148528) (width 0.3) (layer "F.Cu") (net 2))
 (segment (start 86.4 102.9) (end 85.2625 102.9) (width 0.3) (layer "F.Cu") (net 2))
 (segment (start 85.888125 101) (end 85.2625 101) (width 0.3) (layer "F.Cu") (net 2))
 (segment (start 85.975 105.7) (end 86.4 105.7) (width 0.3) (layer "F.Cu") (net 2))
 (segment (start 85.74 104.4) (end 86.4 104.4) (width 0.5) (layer "F.Cu") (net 2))
 (segment (start 86.624264 106.724264) (end 86.575735 106.675735) (width 0.3) (layer "F.Cu") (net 2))
 (segment (start 85.975 105.7) (end 86.4 105.7) (width 0.5) (layer "F.Cu") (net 2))
 (segment (start 86.8 108.9) (end 86.8 106.9) (width 0.5) (layer "F.Cu") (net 2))
 (segment (start 85.74 104.4) (end 86.4 104.4) (width 0.3) (layer "F.Cu") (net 2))
 (segment (start 86.4 106.251471) (end 86.4 101.511875) (width 0.3) (layer "F.Cu") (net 2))
 (arc (start 86.8 107.148528) (mid 86.754327 106.918918) (end 86.624264 106.724264) (width 0.3) (layer "F.Cu") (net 2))
 (arc (start 86.575735 106.675735) (mid 86.445672 106.481081) (end 86.4 106.251471) (width 0.3) (layer "F.Cu") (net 2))
 (arc (start 86.4 101.511875) (mid 86.250075 101.149924) (end 85.888125 101) (width 0.3) (layer "F.Cu") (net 2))
 (segment (start 84.425 105.7) (end 84.2 105.7) (width 0.3) (layer "F.Cu") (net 1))
 (segment (start 86.8 113.5) (end 84.8 113.5) (width 0.3) (layer "F.Cu") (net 1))
 (segment (start 86.8 113.5) (end 86.8 114.3) (width 0.3) (layer "F.Cu") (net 1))
 (segment (start 86.8 113.5) (end 84.2 113.5) (width 0.5) (layer "F.Cu") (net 1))
 (segment (start 88.8 124.671017) (end 90.95 122.671017) (width 0.5) (layer "F.Cu") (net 1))
 (segment (start 84.66 104.4) (end 84.2 104.4) (width 0.5) (layer "F.Cu") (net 1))
 (segment (start 86.025 99.45) (end 84.2 99.45) (width 0.5) (layer "F.Cu") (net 1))
 (segment (start 85.2625 101.95) (end 84.2 101.95) (width 0.3) (layer "F.Cu") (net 1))
 (segment (start 84.8 99.45) (end 86.025 99.45) (width 0.3) (layer "F.Cu") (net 1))
 (segment (start 84.2 112.9) (end 84.2 100.05) (width 0.3) (layer "F.Cu") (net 1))
 (segment (start 84.66 104.4) (end 84.2 104.4) (width 0.3) (layer "F.Cu") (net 1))
 (segment (start 90.758662 122.849005) (end 88.8 124.671017) (width 0.3) (layer "F.Cu") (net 1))
 (segment (start 90.95 115.5) (end 90.95 122.409693) (width 0.3) (layer "F.Cu") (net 1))
 (segment (start 87.399999 114.9) (end 90.35 114.9) (width 0.3) (layer "F.Cu") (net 1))
 (segment (start 86.8 113.5) (end 86.8 114.9) (width 0.5) (layer "F.Cu") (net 1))
 (segment (start 84.425 105.7) (end 84.2 105.7) (width 0.5) (layer "F.Cu") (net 1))
 (arc (start 90.35 114.9) (mid 90.774264 115.075735) (end 90.95 115.5) (width 0.3) (layer "F.Cu") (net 1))
 (arc (start 84.2 100.05) (mid 84.375735 99.625735) (end 84.8 99.45) (width 0.3) (layer "F.Cu") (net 1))
 (arc (start 84.8 113.5) (mid 84.375735 113.324264) (end 84.2 112.9) (width 0.3) (layer "F.Cu") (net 1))
 (arc (start 90.95 122.409693) (mid 90.900089 122.649279) (end 90.758662 122.849005) (width 0.3) (layer "F.Cu") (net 1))
 (arc (start 86.8 114.3) (mid 86.975735 114.724264) (end 87.399999 114.9) (width 0.3) (layer "F.Cu") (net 1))
 (segment (start 88.65 99.93375) (end 88.65 113.5) (width 0.3) (layer "F.Cu") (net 4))
 (segment (start 87.5375 101) (end 87.5375 100.166059) (width 0.3) (layer "F.Cu") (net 4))
 (segment (start 92.65 121.421017) (end 110.6 121.421017) (width 0.3) (layer "F.Cu") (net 4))
 (segment (start 111.2 122.021017) (end 111.2 124.671017) (width 0.3) (layer "F.Cu") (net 4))
 (segment (start 87.538359 100.133963) (end 87.558125 99.765) (width 0.3) (layer "F.Cu") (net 4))
 (segment (start 89.25 114.1) (end 91.45 114.1) (width 0.3) (layer "F.Cu") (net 4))
 (segment (start 87.890451 99.45) (end 88.16625 99.45) (width 0.3) (layer "F.Cu") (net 4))
 (segment (start 111.2 124.671017) (end 111.2 121.421017) (width 0.5) (layer "F.Cu") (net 4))
 (segment (start 92.05 114.7) (end 92.05 120.821017) (width 0.3) (layer "F.Cu") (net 4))
 (arc (start 92.05 120.821017) (mid 92.225735 121.245281) (end 92.65 121.421017) (width 0.3) (layer "F.Cu") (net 4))
 (arc (start 91.45 114.1) (mid 91.874264 114.275735) (end 92.05 114.7) (width 0.3) (layer "F.Cu") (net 4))
 (arc (start 110.6 121.421017) (mid 111.024264 121.596753) (end 111.2 122.021017) (width 0.3) (layer "F.Cu") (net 4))
 (arc (start 88.16625 99.45) (mid 88.508312 99.591687) (end 88.65 99.93375) (width 0.3) (layer "F.Cu") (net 4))
 (arc (start 88.65 113.5) (mid 88.825735 113.924264) (end 89.25 114.1) (width 0.3) (layer "F.Cu") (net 4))
 (arc (start 87.558125 99.765) (mid 87.661505 99.541263) (end 87.890451 99.45) (width 0.3) (layer "F.Cu") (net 4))
 (arc (start 87.5375 100.166059) (mid 87.537714 100.150005) (end 87.538359 100.133963) (width 0.3) (layer "F.Cu") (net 4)))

